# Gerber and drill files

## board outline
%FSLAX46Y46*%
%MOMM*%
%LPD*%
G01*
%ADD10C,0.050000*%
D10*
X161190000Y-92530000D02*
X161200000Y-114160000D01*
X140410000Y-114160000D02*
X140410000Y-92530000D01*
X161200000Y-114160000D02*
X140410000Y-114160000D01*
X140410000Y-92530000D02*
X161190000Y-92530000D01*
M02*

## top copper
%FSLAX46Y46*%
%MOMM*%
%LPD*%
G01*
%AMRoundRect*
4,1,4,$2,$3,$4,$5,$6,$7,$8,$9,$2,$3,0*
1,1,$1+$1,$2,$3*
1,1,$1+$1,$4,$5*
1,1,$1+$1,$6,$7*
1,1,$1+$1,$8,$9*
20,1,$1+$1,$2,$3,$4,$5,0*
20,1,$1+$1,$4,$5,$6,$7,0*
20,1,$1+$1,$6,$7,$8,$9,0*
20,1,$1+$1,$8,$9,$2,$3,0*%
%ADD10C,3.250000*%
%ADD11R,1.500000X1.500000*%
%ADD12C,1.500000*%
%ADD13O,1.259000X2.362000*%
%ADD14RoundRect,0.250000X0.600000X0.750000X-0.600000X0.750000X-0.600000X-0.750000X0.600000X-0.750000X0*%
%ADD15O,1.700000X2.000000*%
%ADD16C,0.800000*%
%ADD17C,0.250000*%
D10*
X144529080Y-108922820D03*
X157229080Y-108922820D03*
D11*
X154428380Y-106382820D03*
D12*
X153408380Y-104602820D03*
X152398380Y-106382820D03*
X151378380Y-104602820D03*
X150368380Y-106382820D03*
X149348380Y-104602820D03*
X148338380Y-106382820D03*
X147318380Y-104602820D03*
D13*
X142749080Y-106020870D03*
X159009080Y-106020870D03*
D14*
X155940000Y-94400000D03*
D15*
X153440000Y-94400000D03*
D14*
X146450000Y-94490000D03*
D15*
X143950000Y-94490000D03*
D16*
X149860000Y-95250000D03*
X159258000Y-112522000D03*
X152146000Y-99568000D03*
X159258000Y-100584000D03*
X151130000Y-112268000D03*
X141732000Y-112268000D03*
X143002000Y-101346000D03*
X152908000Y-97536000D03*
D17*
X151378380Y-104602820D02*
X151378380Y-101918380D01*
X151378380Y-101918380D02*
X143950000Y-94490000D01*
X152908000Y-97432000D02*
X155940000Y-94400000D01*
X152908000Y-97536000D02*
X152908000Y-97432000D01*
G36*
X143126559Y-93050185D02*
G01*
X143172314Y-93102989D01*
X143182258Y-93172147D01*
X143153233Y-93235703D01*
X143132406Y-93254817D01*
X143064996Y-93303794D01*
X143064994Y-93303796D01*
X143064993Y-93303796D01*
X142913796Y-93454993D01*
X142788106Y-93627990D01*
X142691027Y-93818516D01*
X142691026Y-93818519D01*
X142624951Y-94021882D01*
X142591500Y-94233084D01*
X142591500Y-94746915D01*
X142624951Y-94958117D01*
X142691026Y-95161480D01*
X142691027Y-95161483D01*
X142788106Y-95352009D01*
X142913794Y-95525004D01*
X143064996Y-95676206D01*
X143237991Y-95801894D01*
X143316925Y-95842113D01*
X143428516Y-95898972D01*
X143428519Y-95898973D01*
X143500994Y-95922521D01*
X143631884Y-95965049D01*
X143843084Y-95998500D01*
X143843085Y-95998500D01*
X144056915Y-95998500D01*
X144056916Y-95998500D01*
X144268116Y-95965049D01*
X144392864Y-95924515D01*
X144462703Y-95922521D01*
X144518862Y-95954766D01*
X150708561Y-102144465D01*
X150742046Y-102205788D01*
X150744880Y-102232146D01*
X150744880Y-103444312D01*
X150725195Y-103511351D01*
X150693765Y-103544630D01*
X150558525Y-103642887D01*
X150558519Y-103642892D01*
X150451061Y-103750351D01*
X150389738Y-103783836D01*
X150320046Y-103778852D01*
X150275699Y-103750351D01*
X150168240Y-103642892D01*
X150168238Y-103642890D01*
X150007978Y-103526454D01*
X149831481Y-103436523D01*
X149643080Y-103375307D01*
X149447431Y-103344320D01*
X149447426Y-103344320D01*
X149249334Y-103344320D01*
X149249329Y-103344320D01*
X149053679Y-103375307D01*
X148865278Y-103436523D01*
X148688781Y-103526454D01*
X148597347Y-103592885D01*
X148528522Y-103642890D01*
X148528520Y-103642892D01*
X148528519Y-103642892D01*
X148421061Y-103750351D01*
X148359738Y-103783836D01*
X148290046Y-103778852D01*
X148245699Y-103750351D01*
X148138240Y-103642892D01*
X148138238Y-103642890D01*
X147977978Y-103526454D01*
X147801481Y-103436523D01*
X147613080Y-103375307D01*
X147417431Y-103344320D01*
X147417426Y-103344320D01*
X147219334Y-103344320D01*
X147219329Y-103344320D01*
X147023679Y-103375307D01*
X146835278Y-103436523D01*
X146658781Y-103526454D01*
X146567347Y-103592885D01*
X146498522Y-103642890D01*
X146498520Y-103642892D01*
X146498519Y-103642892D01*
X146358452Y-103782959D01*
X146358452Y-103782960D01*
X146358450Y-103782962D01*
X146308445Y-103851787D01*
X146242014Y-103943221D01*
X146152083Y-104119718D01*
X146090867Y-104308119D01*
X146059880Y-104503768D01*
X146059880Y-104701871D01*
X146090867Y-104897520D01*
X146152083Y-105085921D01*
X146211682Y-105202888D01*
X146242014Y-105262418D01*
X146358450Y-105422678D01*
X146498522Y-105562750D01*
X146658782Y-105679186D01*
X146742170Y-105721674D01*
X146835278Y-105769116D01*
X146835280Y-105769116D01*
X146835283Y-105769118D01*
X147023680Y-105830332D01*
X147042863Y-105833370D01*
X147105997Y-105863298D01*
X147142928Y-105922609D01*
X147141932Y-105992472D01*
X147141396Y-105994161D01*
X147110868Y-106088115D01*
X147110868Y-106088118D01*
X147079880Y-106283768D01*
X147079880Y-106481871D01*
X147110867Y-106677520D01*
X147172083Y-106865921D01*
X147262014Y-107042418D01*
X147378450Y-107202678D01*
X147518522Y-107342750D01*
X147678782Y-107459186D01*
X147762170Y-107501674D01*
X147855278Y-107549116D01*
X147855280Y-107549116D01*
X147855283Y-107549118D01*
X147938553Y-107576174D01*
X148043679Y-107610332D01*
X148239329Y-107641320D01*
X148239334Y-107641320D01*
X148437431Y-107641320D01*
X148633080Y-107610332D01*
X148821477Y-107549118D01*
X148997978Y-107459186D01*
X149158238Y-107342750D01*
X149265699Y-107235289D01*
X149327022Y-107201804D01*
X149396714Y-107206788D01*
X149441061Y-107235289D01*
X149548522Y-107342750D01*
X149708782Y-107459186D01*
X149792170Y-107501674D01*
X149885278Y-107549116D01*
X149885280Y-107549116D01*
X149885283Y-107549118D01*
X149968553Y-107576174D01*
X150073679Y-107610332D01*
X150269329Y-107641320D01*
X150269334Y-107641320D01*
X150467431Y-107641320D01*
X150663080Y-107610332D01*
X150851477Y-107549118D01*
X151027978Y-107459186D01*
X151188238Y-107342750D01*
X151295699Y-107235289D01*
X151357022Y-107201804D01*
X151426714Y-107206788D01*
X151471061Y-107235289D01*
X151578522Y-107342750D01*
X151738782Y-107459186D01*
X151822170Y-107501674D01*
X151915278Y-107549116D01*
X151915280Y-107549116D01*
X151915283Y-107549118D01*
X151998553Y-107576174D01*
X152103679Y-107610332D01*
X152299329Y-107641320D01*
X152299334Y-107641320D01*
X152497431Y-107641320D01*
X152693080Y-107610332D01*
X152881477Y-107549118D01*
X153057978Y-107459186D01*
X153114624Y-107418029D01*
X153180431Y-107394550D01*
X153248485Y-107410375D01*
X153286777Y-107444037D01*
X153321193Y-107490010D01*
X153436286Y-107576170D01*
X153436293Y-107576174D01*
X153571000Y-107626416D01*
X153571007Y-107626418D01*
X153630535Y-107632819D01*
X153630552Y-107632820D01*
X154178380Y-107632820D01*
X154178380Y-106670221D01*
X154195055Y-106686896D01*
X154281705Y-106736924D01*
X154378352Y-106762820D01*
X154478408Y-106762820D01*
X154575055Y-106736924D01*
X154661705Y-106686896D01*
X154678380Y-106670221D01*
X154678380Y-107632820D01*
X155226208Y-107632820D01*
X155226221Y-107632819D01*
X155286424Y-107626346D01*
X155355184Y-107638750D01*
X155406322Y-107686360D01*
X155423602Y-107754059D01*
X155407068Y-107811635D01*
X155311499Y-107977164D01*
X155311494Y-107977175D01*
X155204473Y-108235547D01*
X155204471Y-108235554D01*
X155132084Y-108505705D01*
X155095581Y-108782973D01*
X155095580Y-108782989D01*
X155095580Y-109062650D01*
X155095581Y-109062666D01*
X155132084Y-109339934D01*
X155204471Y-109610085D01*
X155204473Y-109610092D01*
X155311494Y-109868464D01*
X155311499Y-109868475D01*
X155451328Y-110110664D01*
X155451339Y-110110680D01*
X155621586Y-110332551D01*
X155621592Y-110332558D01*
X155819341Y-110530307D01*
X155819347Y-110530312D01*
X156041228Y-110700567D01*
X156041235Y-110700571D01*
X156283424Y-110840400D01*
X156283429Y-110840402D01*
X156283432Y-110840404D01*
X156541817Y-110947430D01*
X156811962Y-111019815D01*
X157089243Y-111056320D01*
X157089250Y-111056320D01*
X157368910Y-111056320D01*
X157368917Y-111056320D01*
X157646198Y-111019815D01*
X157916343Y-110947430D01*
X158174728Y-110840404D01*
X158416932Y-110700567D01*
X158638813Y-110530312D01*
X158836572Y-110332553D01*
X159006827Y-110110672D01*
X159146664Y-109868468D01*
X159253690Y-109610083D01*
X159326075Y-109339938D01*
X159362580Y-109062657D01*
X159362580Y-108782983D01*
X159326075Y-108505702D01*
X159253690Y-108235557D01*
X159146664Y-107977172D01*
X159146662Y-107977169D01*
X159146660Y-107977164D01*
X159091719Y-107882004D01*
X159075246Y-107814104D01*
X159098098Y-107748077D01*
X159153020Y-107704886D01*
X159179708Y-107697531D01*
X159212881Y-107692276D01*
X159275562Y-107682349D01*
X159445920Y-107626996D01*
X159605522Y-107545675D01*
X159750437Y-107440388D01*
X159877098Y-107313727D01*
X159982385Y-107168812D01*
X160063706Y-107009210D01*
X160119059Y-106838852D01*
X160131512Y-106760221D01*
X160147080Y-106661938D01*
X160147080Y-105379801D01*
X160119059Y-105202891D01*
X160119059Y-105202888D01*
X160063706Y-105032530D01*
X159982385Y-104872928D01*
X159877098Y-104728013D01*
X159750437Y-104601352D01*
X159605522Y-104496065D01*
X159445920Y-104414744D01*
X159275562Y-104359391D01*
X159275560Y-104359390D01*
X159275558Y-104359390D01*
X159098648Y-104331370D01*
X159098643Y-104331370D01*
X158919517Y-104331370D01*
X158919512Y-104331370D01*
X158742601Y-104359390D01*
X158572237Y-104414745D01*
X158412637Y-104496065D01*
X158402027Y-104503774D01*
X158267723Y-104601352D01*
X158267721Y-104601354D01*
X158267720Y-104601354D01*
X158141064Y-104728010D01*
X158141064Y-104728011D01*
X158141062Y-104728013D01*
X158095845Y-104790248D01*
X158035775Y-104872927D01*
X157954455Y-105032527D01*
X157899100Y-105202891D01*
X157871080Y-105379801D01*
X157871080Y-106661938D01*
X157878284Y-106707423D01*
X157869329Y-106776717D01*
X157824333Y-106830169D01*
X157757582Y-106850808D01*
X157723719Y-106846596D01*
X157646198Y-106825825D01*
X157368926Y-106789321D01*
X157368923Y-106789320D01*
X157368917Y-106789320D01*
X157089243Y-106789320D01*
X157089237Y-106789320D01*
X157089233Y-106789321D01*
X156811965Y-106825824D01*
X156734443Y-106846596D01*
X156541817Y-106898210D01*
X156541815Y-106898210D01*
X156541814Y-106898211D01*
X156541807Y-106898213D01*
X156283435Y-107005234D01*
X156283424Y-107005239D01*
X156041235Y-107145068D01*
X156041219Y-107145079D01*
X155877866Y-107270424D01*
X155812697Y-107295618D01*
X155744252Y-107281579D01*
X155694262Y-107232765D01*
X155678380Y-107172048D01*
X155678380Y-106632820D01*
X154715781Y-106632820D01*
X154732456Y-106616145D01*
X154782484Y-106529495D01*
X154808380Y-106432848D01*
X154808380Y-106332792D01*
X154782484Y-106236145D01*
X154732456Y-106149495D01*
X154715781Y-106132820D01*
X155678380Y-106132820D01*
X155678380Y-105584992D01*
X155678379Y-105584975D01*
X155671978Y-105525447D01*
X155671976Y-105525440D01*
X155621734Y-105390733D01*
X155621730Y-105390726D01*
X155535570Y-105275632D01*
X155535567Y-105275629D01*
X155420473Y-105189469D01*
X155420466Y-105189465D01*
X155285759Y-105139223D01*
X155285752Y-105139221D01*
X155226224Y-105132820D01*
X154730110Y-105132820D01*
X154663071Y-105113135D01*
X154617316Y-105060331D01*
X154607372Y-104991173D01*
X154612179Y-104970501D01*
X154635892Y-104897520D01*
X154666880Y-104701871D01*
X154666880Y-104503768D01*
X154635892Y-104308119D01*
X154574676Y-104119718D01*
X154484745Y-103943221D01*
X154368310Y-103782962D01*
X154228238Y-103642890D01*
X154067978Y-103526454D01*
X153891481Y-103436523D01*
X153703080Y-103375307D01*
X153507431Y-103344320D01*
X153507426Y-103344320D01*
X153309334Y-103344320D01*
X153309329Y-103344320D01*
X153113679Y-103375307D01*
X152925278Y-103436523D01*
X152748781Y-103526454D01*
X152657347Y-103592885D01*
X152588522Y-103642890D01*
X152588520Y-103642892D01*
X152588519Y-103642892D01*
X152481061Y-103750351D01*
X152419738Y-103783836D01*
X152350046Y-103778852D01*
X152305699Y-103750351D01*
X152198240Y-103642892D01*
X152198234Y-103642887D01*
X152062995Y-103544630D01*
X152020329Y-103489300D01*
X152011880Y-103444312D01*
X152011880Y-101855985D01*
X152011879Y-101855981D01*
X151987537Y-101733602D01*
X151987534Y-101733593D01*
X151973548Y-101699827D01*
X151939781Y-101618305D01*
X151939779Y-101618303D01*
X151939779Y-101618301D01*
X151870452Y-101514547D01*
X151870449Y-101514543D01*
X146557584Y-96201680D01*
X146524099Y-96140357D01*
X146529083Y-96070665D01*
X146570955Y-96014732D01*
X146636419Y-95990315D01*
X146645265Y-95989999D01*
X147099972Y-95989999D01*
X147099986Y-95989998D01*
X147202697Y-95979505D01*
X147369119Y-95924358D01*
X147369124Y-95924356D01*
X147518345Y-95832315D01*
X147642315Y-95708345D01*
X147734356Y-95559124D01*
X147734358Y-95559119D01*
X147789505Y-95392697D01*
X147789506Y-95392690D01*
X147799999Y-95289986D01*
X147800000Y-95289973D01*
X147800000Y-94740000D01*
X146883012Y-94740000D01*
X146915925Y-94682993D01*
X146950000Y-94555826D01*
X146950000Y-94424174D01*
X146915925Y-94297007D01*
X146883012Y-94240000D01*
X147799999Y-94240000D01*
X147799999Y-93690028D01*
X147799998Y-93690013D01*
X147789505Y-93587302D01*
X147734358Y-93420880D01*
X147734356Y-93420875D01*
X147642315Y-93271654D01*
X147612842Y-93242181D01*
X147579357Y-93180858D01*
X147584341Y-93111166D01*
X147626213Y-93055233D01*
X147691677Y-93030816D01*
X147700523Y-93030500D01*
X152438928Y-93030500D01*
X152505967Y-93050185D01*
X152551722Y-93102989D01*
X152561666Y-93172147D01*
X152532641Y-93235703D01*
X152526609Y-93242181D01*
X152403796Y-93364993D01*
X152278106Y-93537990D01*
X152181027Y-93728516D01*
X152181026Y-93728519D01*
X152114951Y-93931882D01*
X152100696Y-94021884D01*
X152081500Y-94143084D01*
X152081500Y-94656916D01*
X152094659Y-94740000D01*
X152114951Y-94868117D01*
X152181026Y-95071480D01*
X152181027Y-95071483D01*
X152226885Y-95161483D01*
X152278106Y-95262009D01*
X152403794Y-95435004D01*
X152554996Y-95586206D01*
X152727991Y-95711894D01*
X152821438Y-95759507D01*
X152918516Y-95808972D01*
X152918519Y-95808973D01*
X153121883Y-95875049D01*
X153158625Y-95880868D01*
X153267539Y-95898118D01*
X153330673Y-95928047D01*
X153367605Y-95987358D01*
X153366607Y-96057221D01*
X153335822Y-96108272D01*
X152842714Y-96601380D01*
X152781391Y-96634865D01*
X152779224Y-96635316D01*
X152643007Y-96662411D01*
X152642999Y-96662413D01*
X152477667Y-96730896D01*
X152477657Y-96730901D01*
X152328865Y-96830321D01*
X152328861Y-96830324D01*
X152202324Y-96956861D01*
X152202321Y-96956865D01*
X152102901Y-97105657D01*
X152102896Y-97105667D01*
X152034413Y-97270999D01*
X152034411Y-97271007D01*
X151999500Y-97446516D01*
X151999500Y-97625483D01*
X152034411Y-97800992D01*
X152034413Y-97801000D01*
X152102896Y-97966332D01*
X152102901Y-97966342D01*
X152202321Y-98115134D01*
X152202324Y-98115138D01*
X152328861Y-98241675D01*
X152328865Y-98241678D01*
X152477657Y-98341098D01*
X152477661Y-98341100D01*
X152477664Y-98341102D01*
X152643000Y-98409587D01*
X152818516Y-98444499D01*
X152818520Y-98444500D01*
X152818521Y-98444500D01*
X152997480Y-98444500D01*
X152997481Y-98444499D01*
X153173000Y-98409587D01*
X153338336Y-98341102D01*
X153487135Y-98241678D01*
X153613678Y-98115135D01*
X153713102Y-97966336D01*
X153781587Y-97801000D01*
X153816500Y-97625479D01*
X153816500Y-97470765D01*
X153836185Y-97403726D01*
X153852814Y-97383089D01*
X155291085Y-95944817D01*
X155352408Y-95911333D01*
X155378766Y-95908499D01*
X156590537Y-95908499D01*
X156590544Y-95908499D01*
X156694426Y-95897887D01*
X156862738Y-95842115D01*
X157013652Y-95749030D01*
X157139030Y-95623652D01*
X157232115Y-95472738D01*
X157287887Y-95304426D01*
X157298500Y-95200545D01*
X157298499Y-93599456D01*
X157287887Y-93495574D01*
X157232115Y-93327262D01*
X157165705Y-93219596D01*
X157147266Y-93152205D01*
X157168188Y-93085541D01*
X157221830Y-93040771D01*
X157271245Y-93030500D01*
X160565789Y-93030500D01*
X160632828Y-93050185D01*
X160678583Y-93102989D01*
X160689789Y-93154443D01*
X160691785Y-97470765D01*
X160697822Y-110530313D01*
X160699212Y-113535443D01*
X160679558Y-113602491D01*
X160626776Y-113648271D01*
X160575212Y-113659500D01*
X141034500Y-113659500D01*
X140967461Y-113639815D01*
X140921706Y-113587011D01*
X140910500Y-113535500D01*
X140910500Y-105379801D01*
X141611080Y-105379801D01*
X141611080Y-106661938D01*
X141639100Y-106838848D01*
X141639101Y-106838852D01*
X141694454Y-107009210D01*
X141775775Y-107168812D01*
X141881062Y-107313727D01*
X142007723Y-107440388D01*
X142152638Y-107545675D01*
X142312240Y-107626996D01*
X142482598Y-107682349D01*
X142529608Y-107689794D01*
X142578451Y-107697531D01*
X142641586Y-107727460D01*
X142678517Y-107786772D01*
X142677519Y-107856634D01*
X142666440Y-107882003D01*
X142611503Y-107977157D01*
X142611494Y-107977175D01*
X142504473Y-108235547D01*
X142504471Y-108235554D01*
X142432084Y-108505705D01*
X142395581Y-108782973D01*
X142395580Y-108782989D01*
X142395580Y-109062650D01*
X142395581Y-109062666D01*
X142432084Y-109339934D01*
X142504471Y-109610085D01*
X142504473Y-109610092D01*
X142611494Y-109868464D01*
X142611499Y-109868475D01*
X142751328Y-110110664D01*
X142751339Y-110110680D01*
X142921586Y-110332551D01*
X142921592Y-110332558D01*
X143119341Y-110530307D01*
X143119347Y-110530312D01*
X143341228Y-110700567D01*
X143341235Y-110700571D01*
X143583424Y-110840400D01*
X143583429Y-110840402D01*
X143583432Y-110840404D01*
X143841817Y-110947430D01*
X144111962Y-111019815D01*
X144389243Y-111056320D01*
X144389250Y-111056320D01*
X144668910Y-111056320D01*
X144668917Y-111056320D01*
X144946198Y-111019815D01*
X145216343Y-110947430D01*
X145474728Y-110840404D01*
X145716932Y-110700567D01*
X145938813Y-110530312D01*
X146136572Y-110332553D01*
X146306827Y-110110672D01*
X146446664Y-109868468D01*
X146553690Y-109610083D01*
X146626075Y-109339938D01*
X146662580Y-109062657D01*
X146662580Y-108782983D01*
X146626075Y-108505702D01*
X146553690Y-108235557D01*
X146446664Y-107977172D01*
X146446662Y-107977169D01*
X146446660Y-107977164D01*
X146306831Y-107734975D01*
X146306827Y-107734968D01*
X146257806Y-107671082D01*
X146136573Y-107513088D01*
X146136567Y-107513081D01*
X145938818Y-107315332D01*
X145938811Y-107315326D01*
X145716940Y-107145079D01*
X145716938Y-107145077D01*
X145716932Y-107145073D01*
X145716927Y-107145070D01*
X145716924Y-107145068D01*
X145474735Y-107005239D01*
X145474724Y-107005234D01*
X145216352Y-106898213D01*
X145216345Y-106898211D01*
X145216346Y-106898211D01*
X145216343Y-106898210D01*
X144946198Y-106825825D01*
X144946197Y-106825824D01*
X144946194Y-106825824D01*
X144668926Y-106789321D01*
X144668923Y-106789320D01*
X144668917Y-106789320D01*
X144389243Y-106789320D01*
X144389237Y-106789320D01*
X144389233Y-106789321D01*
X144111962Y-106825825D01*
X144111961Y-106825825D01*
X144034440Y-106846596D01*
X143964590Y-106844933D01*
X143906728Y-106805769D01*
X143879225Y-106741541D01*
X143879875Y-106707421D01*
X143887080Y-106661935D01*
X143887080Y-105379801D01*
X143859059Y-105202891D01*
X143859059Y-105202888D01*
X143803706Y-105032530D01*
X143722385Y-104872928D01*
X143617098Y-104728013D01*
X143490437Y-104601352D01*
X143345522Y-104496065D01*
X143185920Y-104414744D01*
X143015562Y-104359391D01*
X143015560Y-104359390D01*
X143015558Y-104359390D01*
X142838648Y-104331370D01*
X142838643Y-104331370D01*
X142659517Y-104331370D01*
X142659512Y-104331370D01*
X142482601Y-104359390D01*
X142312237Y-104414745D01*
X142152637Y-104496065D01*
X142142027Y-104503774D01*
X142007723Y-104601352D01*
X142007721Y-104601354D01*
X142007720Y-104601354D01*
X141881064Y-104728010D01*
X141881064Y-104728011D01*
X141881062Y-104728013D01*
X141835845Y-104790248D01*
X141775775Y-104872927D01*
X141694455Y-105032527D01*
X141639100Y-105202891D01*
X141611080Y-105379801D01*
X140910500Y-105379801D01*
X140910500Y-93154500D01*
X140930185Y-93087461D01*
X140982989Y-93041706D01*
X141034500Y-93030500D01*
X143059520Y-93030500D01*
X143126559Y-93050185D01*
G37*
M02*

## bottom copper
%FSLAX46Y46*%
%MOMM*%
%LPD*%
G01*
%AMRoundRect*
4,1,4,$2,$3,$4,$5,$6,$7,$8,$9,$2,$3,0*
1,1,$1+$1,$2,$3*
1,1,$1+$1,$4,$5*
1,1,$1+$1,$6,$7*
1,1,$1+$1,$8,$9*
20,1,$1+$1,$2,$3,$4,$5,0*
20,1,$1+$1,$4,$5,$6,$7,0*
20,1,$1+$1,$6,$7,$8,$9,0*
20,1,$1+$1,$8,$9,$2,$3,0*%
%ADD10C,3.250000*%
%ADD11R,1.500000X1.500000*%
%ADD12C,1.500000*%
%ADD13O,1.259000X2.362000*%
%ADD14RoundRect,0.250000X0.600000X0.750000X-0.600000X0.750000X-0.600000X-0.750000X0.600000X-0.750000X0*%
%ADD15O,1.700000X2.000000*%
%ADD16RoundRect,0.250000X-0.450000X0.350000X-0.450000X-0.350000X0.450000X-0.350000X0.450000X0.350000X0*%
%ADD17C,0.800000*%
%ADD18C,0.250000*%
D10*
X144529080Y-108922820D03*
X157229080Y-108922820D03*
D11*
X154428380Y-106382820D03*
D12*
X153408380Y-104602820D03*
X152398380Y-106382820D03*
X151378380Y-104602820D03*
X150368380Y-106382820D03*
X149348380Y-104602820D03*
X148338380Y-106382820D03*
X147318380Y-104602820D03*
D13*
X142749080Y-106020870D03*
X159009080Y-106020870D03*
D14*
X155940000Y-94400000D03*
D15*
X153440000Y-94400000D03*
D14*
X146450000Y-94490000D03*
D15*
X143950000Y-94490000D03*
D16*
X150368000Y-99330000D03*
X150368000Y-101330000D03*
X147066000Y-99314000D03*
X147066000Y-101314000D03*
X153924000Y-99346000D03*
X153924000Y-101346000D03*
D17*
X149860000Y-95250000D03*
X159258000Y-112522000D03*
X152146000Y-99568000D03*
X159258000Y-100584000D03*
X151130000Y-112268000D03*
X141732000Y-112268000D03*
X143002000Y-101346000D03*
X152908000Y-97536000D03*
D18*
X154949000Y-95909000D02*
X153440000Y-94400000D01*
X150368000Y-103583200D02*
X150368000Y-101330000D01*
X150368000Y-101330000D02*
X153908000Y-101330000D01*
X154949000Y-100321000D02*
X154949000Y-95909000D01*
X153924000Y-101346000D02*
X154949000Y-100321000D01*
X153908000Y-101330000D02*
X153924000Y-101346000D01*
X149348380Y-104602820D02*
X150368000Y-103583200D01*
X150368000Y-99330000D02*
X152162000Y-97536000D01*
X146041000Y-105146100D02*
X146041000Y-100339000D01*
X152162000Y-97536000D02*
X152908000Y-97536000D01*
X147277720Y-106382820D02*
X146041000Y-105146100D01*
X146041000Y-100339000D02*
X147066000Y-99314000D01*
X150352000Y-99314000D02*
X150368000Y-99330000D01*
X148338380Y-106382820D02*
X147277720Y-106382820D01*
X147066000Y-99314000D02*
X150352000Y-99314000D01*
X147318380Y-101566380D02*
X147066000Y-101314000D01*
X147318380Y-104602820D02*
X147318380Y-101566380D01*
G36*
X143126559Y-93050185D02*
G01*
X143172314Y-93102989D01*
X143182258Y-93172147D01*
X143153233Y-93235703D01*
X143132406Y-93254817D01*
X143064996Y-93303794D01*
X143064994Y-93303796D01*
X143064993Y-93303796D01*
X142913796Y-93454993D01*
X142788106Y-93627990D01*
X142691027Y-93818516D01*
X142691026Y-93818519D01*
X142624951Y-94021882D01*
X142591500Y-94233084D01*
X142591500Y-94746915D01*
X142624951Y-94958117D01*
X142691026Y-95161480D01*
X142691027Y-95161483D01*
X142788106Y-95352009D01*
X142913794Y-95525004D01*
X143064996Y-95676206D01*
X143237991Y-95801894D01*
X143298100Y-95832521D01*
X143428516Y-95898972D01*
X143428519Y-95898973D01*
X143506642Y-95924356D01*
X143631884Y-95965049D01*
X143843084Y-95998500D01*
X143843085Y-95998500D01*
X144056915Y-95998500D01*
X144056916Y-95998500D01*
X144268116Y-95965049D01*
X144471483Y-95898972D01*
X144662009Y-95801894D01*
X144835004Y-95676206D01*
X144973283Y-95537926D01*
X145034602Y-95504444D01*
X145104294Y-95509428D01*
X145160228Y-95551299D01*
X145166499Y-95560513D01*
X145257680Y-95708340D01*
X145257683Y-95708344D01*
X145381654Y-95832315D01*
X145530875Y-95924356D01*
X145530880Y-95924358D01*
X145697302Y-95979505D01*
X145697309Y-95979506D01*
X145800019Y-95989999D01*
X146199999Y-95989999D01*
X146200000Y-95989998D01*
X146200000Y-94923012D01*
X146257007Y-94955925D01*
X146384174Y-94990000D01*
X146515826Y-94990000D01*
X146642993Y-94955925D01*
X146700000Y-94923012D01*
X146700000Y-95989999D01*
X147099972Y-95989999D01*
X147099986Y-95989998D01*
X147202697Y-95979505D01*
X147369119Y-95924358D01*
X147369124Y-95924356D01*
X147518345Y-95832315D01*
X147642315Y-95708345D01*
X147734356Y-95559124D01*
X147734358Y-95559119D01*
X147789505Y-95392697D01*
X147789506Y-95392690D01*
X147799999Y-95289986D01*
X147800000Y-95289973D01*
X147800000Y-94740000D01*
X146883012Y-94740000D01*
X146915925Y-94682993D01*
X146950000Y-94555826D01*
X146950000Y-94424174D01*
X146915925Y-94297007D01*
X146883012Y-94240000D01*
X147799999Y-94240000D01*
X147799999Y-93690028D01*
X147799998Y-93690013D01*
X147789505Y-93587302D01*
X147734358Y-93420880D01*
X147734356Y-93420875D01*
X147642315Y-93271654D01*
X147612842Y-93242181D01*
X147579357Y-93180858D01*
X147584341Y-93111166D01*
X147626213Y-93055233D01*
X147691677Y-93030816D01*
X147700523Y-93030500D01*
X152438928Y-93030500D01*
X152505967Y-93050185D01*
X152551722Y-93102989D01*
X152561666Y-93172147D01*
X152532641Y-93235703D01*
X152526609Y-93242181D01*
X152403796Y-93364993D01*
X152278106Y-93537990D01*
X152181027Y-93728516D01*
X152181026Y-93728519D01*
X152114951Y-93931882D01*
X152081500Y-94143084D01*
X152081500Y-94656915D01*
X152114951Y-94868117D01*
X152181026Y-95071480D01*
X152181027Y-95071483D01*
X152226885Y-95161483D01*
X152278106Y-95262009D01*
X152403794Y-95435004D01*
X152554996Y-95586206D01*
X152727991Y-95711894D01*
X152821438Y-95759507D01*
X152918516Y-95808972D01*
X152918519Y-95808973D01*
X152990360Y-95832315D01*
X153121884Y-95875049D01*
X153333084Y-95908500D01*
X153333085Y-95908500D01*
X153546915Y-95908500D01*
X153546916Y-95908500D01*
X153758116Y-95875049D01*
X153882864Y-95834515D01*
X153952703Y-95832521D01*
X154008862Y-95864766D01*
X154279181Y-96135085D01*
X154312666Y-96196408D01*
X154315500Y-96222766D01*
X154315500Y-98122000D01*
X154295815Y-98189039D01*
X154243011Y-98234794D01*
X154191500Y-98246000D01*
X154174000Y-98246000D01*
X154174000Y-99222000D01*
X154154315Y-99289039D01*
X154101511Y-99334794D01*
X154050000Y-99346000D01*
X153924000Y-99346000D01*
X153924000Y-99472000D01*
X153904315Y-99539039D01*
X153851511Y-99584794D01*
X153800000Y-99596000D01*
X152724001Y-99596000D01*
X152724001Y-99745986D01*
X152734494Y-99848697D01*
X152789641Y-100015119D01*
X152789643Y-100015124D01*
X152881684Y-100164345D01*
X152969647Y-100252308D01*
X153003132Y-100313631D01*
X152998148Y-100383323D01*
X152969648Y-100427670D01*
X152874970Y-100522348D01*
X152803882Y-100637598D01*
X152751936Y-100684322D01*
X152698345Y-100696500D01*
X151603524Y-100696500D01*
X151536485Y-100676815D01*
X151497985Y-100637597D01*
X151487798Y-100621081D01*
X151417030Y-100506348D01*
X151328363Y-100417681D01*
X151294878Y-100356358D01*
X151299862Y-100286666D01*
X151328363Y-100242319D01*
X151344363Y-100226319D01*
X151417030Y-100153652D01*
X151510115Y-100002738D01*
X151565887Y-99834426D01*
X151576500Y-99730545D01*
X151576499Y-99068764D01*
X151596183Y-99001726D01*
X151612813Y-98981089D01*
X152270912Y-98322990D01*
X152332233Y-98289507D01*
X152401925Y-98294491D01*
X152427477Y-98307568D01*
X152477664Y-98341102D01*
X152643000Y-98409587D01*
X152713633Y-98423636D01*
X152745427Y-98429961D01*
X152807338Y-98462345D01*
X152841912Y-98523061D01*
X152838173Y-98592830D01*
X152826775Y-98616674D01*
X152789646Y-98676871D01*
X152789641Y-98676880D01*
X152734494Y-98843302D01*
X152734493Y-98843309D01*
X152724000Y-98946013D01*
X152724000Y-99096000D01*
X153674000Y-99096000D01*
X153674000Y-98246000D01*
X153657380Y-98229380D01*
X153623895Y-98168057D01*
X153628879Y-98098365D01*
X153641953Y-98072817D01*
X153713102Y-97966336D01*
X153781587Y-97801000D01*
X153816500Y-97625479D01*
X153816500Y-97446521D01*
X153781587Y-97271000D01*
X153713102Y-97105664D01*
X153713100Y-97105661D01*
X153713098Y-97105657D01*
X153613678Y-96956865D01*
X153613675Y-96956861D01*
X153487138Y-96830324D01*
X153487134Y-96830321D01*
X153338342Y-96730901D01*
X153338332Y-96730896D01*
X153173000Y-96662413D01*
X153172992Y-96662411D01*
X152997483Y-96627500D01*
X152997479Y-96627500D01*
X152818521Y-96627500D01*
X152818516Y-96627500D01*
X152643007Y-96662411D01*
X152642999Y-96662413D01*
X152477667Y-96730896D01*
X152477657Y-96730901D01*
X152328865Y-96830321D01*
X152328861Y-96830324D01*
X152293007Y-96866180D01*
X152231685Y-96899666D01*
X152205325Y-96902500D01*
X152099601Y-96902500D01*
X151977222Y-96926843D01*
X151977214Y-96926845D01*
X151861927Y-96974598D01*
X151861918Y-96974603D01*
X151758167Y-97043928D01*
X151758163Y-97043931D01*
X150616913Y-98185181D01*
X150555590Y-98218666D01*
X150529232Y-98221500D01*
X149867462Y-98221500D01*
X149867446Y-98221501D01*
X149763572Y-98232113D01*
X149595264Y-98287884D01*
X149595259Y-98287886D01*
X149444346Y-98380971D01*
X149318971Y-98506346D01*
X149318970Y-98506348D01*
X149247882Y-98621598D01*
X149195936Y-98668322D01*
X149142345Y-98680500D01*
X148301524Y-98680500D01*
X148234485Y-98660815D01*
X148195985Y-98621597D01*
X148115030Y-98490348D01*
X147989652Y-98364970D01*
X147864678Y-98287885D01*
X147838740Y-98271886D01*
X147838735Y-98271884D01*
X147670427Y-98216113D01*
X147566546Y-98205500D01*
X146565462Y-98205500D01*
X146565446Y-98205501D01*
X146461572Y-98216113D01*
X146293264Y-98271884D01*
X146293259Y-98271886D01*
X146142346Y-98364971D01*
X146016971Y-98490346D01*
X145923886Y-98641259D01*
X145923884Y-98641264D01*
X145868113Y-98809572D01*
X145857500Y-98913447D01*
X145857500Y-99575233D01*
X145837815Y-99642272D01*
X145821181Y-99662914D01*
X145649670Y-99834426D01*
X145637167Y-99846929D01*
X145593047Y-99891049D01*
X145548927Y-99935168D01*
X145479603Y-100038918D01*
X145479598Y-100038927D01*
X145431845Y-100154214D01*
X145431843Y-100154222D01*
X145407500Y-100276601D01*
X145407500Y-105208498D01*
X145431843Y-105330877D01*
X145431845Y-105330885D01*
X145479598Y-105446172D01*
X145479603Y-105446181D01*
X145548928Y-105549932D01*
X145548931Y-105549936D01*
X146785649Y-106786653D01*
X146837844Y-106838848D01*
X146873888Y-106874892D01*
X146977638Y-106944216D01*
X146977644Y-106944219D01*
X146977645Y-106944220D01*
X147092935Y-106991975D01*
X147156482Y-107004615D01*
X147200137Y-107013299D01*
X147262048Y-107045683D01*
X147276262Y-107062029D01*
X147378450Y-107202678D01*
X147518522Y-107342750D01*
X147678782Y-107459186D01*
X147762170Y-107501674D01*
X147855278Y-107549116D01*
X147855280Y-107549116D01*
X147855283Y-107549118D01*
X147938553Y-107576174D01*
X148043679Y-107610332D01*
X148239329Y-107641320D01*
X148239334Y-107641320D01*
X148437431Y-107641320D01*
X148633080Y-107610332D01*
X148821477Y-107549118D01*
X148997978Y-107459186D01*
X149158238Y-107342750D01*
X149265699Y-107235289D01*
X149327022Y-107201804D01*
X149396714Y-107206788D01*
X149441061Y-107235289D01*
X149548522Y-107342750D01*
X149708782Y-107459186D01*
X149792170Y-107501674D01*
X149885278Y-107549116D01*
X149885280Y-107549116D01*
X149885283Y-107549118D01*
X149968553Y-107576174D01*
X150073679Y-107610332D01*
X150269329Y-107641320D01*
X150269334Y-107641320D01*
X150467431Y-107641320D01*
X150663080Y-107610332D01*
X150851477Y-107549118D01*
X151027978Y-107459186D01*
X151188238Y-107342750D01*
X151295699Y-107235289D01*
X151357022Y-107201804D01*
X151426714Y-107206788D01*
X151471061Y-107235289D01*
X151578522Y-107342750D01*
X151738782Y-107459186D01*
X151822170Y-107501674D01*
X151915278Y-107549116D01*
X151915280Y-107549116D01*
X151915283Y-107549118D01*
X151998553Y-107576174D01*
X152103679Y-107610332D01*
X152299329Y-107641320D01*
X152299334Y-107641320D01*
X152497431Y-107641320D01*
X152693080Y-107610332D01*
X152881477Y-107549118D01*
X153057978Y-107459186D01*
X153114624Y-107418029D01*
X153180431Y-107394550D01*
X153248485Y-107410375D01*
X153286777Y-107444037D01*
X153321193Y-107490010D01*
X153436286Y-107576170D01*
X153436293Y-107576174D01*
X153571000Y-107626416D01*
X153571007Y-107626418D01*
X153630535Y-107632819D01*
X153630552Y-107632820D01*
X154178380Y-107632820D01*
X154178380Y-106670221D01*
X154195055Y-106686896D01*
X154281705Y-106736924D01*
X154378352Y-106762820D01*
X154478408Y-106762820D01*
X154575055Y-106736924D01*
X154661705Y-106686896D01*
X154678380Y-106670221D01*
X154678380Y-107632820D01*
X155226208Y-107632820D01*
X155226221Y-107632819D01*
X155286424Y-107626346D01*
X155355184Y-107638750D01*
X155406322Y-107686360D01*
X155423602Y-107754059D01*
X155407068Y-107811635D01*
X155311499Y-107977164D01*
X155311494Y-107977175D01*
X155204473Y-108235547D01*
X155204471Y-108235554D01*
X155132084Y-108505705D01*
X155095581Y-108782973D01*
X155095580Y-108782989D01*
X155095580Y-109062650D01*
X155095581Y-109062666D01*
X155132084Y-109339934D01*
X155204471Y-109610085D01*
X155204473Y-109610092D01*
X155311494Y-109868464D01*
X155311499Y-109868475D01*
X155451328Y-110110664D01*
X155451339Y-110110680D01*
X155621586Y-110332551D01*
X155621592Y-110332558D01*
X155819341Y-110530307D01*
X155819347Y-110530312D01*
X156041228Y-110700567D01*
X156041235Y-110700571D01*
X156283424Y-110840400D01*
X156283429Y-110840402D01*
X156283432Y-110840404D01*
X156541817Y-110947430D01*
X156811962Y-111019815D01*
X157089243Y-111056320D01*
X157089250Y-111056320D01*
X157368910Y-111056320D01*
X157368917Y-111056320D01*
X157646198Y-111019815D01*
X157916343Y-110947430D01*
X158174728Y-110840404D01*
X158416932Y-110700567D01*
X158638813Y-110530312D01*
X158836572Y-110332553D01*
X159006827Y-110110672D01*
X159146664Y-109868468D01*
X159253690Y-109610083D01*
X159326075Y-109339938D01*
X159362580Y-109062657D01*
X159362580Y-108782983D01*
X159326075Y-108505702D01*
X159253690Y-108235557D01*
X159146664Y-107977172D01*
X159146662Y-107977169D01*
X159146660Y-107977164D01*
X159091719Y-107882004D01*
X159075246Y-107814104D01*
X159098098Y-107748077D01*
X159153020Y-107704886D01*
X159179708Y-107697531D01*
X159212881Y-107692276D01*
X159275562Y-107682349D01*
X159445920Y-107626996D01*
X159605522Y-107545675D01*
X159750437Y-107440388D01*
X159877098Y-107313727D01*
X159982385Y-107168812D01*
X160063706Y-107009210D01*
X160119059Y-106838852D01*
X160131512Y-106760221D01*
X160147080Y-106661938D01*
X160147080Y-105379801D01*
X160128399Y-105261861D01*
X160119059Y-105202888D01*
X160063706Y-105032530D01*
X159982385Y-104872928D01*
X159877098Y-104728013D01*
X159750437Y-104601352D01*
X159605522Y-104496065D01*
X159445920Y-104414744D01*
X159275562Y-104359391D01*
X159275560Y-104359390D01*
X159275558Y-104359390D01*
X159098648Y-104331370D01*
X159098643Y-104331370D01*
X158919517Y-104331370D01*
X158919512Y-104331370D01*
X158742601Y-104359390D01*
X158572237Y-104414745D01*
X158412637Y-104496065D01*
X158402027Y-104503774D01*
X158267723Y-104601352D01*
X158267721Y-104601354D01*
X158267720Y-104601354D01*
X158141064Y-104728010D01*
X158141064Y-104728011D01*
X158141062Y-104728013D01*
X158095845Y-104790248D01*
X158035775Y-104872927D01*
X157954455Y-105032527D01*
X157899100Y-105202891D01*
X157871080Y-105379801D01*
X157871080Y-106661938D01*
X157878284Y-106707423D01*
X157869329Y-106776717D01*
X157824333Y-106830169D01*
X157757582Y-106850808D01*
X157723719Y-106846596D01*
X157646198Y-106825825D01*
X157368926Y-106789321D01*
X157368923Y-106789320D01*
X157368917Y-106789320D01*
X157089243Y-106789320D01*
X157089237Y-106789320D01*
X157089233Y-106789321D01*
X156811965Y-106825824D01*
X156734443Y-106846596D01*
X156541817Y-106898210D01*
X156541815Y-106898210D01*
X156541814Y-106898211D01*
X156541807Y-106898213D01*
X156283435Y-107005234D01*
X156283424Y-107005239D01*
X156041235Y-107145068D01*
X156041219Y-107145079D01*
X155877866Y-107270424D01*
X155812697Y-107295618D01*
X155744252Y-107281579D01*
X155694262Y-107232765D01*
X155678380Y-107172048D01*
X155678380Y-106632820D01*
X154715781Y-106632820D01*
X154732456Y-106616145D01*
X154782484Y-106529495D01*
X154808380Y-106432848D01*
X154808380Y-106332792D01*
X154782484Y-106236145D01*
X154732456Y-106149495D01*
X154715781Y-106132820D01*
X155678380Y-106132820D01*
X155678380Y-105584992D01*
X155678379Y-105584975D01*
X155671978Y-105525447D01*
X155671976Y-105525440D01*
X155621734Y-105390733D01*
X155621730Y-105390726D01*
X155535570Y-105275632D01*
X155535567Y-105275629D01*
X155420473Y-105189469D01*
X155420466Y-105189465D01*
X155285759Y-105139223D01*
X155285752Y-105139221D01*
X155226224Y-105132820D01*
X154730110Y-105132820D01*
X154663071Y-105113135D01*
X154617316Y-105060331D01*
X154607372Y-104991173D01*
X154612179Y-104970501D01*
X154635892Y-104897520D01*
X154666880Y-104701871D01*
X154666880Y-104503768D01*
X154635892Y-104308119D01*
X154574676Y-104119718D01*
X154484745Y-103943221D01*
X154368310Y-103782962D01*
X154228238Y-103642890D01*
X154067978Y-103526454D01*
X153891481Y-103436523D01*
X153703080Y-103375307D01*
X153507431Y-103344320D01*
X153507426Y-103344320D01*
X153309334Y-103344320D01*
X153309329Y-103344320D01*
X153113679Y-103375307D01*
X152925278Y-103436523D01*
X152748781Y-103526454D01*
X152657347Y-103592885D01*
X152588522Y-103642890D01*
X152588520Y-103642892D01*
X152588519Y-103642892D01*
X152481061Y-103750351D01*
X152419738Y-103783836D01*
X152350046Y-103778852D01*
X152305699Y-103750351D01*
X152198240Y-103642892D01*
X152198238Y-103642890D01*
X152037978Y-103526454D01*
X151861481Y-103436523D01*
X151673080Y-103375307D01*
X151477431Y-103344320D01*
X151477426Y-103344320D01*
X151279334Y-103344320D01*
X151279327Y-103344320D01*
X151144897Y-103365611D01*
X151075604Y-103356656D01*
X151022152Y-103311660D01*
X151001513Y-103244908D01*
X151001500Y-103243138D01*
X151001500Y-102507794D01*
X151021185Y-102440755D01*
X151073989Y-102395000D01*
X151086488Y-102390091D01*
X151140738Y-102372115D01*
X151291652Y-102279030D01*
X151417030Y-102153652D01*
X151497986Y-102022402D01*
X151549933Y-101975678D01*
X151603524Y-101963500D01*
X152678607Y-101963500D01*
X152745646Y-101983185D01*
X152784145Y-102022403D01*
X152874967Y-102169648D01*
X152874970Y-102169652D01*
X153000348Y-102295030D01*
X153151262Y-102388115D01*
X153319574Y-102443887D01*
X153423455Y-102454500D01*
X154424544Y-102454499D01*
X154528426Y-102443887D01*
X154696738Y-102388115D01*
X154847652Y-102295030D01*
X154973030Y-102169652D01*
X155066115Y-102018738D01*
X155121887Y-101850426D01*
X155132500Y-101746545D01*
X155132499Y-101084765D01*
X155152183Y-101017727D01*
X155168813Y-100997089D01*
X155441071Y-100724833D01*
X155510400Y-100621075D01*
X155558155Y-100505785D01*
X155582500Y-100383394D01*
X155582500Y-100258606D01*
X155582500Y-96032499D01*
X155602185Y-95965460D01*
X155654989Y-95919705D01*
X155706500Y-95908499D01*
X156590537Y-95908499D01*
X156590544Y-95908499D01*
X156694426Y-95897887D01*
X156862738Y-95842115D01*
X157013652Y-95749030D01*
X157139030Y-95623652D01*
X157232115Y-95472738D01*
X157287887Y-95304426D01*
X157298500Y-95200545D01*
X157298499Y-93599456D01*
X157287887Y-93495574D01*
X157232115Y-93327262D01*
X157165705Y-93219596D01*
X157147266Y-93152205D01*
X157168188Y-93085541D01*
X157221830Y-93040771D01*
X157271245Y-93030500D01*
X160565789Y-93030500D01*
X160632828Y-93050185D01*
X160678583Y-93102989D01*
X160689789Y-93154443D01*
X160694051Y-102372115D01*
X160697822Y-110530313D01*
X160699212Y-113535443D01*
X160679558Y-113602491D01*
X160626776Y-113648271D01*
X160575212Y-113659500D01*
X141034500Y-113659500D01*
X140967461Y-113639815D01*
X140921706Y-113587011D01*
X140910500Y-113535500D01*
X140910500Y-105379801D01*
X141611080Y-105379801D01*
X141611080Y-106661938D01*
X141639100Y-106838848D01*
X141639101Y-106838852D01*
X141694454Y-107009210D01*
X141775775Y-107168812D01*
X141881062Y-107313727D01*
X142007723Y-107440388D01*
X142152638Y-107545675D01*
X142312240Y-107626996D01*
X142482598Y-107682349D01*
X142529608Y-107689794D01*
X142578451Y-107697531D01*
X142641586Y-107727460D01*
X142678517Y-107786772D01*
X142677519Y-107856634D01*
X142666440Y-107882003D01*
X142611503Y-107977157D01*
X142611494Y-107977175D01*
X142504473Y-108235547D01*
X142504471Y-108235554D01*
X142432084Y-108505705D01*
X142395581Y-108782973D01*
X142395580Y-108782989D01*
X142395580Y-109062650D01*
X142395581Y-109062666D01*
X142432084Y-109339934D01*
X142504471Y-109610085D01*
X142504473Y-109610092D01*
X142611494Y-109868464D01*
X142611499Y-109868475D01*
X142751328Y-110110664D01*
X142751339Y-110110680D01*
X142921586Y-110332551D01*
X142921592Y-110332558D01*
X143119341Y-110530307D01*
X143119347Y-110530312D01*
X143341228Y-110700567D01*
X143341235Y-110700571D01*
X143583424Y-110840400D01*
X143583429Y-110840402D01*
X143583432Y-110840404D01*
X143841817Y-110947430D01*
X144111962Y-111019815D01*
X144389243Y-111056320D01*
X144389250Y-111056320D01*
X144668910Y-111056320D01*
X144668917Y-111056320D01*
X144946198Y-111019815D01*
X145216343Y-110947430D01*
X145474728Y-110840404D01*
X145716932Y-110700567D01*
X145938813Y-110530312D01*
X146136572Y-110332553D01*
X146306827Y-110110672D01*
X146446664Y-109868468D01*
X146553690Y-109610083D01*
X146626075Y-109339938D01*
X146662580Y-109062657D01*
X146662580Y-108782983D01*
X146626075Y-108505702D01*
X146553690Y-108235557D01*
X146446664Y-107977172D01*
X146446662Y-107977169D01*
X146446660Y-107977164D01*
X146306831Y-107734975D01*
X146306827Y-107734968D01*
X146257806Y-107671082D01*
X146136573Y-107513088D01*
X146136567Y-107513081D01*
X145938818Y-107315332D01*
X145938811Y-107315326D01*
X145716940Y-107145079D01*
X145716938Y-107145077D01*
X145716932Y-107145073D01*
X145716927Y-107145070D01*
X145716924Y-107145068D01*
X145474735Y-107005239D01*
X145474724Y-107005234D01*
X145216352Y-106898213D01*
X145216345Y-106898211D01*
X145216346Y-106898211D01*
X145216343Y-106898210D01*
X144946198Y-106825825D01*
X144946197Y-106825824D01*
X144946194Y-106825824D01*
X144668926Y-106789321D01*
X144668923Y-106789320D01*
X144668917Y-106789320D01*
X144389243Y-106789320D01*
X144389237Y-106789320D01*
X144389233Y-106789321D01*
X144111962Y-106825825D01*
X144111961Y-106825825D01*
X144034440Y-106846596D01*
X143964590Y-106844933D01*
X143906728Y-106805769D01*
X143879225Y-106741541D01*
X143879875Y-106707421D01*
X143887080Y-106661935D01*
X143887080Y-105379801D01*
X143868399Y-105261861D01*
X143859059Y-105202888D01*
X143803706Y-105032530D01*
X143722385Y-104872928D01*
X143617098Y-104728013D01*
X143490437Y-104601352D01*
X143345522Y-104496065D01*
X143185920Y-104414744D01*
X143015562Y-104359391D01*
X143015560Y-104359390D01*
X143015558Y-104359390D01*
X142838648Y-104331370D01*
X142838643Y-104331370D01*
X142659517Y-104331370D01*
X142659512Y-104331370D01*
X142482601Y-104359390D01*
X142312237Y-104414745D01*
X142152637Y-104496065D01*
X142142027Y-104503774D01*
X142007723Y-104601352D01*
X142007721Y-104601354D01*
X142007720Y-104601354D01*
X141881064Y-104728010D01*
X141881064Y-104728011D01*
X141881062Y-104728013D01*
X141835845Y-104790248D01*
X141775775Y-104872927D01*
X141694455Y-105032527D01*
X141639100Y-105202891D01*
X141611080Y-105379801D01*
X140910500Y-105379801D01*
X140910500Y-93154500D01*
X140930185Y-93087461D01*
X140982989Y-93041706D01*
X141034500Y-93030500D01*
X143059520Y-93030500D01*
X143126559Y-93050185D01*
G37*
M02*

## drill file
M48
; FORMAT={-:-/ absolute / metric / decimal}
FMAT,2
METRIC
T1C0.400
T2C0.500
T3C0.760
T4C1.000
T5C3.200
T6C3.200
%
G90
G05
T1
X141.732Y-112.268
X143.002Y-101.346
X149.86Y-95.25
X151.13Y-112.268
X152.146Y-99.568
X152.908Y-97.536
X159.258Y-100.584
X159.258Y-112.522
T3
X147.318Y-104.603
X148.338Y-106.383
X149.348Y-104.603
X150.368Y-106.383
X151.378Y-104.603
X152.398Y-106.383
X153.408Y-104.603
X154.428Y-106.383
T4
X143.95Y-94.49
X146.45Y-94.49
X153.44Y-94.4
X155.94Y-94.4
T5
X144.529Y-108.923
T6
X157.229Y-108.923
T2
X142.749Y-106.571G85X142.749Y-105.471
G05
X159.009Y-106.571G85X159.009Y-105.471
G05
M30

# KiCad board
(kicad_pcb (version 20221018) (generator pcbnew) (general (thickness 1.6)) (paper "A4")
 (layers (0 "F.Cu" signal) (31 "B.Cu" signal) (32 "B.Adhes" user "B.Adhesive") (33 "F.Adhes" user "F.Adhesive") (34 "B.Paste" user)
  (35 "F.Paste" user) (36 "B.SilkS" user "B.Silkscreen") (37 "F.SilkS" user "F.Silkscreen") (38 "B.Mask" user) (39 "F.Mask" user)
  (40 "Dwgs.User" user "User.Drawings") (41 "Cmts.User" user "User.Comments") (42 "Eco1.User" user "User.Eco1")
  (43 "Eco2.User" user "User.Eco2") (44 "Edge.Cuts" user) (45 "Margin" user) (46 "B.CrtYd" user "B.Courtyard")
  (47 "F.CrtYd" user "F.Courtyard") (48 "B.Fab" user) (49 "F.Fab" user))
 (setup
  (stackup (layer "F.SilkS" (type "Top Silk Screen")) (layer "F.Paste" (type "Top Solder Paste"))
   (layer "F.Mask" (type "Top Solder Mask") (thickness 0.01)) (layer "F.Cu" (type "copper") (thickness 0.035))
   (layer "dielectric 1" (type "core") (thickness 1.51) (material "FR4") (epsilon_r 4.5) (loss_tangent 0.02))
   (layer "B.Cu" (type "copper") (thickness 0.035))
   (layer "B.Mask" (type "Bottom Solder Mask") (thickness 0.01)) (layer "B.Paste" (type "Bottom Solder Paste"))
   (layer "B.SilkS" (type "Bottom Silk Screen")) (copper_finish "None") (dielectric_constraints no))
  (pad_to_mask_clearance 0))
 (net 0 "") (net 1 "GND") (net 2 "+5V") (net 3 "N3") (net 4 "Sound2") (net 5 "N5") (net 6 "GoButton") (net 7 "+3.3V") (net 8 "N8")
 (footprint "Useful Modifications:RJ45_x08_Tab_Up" (layer "F.Cu") (at 150.6474 109.982)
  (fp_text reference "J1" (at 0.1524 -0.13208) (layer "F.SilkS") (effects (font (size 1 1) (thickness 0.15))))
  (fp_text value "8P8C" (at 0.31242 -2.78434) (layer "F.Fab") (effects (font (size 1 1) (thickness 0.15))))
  (pad "" np_thru_hole circle (at -6.11832 -1.05918 180) (size 3.25 3.25) (drill 3.2) (layers "*.Cu" "*.Mask"))
  (pad "" np_thru_hole circle (at 6.58168 -1.05918 180) (size 3.25 3.25) (drill 3.200001) (layers "*.Cu" "*.Mask"))
  (pad "1" thru_hole rect (at 3.78098 -3.59918) (size 1.5 1.5) (drill 0.76) (layers "*.Cu" "*.Mask") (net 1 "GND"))
  (pad "2" thru_hole circle (at 2.76098 -5.37918) (size 1.5 1.5) (drill 0.76) (layers "*.Cu" "*.Mask") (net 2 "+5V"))
  (pad "3" thru_hole circle (at 1.75098 -3.59918) (size 1.5 1.5) (drill 0.76) (layers "*.Cu" "*.Mask") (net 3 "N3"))
  (pad "4" thru_hole circle (at 0.73098 -5.37918) (size 1.5 1.5) (drill 0.76) (layers "*.Cu" "*.Mask") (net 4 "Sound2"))
  (pad "5" thru_hole circle (at -0.27902 -3.59918) (size 1.5 1.5) (drill 0.76) (layers "*.Cu" "*.Mask") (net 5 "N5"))
  (pad "6" thru_hole circle (at -1.29902 -5.37918) (size 1.5 1.5) (drill 0.76) (layers "*.Cu" "*.Mask") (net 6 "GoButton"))
  (pad "7" thru_hole circle (at -2.30902 -3.59918) (size 1.5 1.5) (drill 0.76) (layers "*.Cu" "*.Mask") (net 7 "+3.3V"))
  (pad "8" thru_hole circle (at -3.32902 -5.37918) (size 1.5 1.5) (drill 0.76) (layers "*.Cu" "*.Mask") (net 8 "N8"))
  (pad "9" thru_hole oval (at -7.89832 -3.96113 180) (size 1.259 2.362) (drill oval 0.5 1.6) (layers "*.Cu" "*.Mask"))
  (pad "10" thru_hole oval (at 8.36168 -3.96113 180) (size 1.259 2.362) (drill oval 0.5 1.6) (layers "*.Cu" "*.Mask")))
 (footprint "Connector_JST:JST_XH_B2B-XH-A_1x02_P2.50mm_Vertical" (layer "F.Cu") (at 155.94 94.4 180)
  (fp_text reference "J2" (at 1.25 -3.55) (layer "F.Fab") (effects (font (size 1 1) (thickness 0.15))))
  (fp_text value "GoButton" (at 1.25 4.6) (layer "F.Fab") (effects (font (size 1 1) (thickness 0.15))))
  (pad "1" thru_hole roundrect (at 0 0 180) (size 1.7 2) (drill 1) (layers "*.Cu" "*.Mask") (roundrect_rratio 0.1470588235) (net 7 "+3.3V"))
  (pad "2" thru_hole oval (at 2.5 0 180) (size 1.7 2) (drill 1) (layers "*.Cu" "*.Mask") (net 6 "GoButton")))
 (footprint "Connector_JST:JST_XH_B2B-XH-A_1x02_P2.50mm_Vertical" (layer "F.Cu") (at 146.45 94.49 180)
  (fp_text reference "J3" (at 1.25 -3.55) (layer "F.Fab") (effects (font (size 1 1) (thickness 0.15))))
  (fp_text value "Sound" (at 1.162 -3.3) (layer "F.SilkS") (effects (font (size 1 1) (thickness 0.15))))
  (pad "1" thru_hole roundrect (at 0 0 180) (size 1.7 2) (drill 1) (layers "*.Cu" "*.Mask") (roundrect_rratio 0.1470588235) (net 1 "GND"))
  (pad "2" thru_hole oval (at 2.5 0 180) (size 1.7 2) (drill 1) (layers "*.Cu" "*.Mask") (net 4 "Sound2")))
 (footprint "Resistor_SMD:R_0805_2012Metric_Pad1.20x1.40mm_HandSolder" (layer "B.Cu") (at 150.368 100.33 -90)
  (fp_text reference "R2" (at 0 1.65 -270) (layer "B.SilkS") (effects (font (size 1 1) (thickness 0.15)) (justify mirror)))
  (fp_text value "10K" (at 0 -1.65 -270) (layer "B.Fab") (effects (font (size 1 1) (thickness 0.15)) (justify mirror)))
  (pad "1" smd roundrect (at -1 0 270) (size 1.2 1.4) (layers "B.Cu" "B.Paste" "B.Mask") (roundrect_rratio 0.2083333333) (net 7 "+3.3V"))
  (pad "2" smd roundrect (at 1 0 270) (size 1.2 1.4) (layers "B.Cu" "B.Paste" "B.Mask") (roundrect_rratio 0.2083333333) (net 6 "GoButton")))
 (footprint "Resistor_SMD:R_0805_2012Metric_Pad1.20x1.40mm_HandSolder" (layer "B.Cu") (at 147.066 100.314 -90)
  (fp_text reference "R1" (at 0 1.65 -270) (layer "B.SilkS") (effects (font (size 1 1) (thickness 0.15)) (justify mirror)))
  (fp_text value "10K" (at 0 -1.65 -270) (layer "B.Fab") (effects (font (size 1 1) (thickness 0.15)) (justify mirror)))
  (pad "1" smd roundrect (at -1 0 270) (size 1.2 1.4) (layers "B.Cu" "B.Paste" "B.Mask") (roundrect_rratio 0.2083333333) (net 7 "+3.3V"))
  (pad "2" smd roundrect (at 1 0 270) (size 1.2 1.4) (layers "B.Cu" "B.Paste" "B.Mask") (roundrect_rratio 0.2083333333) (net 8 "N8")))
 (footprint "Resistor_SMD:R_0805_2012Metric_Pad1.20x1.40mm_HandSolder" (layer "B.Cu") (at 153.924 100.346 -90)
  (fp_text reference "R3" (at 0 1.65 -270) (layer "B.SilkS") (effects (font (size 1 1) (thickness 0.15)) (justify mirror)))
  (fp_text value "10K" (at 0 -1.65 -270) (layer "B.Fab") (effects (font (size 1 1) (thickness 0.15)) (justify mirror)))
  (pad "1" smd roundrect (at -1 0 270) (size 1.2 1.4) (layers "B.Cu" "B.Paste" "B.Mask") (roundrect_rratio 0.2083333333) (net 1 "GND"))
  (pad "2" smd roundrect (at 1 0 270) (size 1.2 1.4) (layers "B.Cu" "B.Paste" "B.Mask") (roundrect_rratio 0.2083333333) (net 6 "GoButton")))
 (gr_line (start 161.19 92.53) (end 161.2 114.16) (stroke (width 0.05) (type solid)) (layer "Edge.Cuts"))
 (gr_line (start 140.41 114.16) (end 140.41 92.53) (stroke (width 0.05) (type solid)) (layer "Edge.Cuts"))
 (gr_line (start 161.2 114.16) (end 140.41 114.16) (stroke (width 0.05) (type solid)) (layer "Edge.Cuts"))
 (gr_line (start 140.41 92.53) (end 161.19 92.53) (stroke (width 0.05) (type solid)) (layer "Edge.Cuts"))
 (via (at 149.86 95.25) (size 0.8) (drill 0.4) (layers "F.Cu" "B.Cu") (free) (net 1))
 (via (at 159.258 112.522) (size 0.8) (drill 0.4) (layers "F.Cu" "B.Cu") (free) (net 1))
 (via (at 152.146 99.568) (size 0.8) (drill 0.4) (layers "F.Cu" "B.Cu") (free) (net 1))
 (via (at 159.258 100.584) (size 0.8) (drill 0.4) (layers "F.Cu" "B.Cu") (free) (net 1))
 (via (at 151.13 112.268) (size 0.8) (drill 0.4) (layers "F.Cu" "B.Cu") (free) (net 1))
 (via (at 141.732 112.268) (size 0.8) (drill 0.4) (layers "F.Cu" "B.Cu") (free) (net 1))
 (via (at 143.002 101.346) (size 0.8) (drill 0.4) (layers "F.Cu" "B.Cu") (free) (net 1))
 (segment (start 151.37838 104.60282) (end 151.37838 101.91838) (width 0.25) (layer "F.Cu") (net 4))
 (segment (start 151.37838 101.91838) (end 143.95 94.49) (width 0.25) (layer "F.Cu") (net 4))
 (segment (start 154.949 95.909) (end 153.44 94.4) (width 0.25) (layer "B.Cu") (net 6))
 (segment (start 150.368 103.5832) (end 150.368 101.33) (width 0.25) (layer "B.Cu") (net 6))
 (segment (start 150.368 101.33) (end 153.908 101.33) (width 0.25) (layer "B.Cu") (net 6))
 (segment (start 154.949 100.321) (end 154.949 95.909) (width 0.25) (layer "B.Cu") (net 6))
 (segment (start 153.924 101.346) (end 154.949 100.321) (width 0.25) (layer "B.Cu") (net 6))
 (segment (start 153.908 101.33) (end 153.924 101.346) (width 0.25) (layer "B.Cu") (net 6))
 (segment (start 149.34838 104.60282) (end 150.368 103.5832) (width 0.25) (layer "B.Cu") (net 6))
 (segment (start 152.908 97.432) (end 155.94 94.4) (width 0.25) (layer "F.Cu") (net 7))
 (segment (start 152.908 97.536) (end 152.908 97.432) (width 0.25) (layer "F.Cu") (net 7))
 (via (at 152.908 97.536) (size 0.8) (drill 0.4) (layers "F.Cu" "B.Cu") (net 7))
 (segment (start 150.368 99.33) (end 152.162 97.536) (width 0.25) (layer "B.Cu") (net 7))
 (segment (start 146.041 105.1461) (end 146.041 100.339) (width 0.25) (layer "B.Cu") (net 7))
 (segment (start 152.162 97.536) (end 152.908 97.536) (width 0.25) (layer "B.Cu") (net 7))
 (segment (start 147.27772 106.38282) (end 146.041 105.1461) (width 0.25) (layer "B.Cu") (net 7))
 (segment (start 146.041 100.339) (end 147.066 99.314) (width 0.25) (layer "B.Cu") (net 7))
 (segment (start 150.352 99.314) (end 150.368 99.33) (width 0.25) (layer "B.Cu") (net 7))
 (segment (start 148.33838 106.38282) (end 147.27772 106.38282) (width 0.25) (layer "B.Cu") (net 7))
 (segment (start 147.066 99.314) (end 150.352 99.314) (width 0.25) (layer "B.Cu") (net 7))
 (segment (start 147.31838 101.56638) (end 147.066 101.314) (width 0.25) (layer "B.Cu") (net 8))
 (segment (start 147.31838 104.60282) (end 147.31838 101.56638) (width 0.25) (layer "B.Cu") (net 8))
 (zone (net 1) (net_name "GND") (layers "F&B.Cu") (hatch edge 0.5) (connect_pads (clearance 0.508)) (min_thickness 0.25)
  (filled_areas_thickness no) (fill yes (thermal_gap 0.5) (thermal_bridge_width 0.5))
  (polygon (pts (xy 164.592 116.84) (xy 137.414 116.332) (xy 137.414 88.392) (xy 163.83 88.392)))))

